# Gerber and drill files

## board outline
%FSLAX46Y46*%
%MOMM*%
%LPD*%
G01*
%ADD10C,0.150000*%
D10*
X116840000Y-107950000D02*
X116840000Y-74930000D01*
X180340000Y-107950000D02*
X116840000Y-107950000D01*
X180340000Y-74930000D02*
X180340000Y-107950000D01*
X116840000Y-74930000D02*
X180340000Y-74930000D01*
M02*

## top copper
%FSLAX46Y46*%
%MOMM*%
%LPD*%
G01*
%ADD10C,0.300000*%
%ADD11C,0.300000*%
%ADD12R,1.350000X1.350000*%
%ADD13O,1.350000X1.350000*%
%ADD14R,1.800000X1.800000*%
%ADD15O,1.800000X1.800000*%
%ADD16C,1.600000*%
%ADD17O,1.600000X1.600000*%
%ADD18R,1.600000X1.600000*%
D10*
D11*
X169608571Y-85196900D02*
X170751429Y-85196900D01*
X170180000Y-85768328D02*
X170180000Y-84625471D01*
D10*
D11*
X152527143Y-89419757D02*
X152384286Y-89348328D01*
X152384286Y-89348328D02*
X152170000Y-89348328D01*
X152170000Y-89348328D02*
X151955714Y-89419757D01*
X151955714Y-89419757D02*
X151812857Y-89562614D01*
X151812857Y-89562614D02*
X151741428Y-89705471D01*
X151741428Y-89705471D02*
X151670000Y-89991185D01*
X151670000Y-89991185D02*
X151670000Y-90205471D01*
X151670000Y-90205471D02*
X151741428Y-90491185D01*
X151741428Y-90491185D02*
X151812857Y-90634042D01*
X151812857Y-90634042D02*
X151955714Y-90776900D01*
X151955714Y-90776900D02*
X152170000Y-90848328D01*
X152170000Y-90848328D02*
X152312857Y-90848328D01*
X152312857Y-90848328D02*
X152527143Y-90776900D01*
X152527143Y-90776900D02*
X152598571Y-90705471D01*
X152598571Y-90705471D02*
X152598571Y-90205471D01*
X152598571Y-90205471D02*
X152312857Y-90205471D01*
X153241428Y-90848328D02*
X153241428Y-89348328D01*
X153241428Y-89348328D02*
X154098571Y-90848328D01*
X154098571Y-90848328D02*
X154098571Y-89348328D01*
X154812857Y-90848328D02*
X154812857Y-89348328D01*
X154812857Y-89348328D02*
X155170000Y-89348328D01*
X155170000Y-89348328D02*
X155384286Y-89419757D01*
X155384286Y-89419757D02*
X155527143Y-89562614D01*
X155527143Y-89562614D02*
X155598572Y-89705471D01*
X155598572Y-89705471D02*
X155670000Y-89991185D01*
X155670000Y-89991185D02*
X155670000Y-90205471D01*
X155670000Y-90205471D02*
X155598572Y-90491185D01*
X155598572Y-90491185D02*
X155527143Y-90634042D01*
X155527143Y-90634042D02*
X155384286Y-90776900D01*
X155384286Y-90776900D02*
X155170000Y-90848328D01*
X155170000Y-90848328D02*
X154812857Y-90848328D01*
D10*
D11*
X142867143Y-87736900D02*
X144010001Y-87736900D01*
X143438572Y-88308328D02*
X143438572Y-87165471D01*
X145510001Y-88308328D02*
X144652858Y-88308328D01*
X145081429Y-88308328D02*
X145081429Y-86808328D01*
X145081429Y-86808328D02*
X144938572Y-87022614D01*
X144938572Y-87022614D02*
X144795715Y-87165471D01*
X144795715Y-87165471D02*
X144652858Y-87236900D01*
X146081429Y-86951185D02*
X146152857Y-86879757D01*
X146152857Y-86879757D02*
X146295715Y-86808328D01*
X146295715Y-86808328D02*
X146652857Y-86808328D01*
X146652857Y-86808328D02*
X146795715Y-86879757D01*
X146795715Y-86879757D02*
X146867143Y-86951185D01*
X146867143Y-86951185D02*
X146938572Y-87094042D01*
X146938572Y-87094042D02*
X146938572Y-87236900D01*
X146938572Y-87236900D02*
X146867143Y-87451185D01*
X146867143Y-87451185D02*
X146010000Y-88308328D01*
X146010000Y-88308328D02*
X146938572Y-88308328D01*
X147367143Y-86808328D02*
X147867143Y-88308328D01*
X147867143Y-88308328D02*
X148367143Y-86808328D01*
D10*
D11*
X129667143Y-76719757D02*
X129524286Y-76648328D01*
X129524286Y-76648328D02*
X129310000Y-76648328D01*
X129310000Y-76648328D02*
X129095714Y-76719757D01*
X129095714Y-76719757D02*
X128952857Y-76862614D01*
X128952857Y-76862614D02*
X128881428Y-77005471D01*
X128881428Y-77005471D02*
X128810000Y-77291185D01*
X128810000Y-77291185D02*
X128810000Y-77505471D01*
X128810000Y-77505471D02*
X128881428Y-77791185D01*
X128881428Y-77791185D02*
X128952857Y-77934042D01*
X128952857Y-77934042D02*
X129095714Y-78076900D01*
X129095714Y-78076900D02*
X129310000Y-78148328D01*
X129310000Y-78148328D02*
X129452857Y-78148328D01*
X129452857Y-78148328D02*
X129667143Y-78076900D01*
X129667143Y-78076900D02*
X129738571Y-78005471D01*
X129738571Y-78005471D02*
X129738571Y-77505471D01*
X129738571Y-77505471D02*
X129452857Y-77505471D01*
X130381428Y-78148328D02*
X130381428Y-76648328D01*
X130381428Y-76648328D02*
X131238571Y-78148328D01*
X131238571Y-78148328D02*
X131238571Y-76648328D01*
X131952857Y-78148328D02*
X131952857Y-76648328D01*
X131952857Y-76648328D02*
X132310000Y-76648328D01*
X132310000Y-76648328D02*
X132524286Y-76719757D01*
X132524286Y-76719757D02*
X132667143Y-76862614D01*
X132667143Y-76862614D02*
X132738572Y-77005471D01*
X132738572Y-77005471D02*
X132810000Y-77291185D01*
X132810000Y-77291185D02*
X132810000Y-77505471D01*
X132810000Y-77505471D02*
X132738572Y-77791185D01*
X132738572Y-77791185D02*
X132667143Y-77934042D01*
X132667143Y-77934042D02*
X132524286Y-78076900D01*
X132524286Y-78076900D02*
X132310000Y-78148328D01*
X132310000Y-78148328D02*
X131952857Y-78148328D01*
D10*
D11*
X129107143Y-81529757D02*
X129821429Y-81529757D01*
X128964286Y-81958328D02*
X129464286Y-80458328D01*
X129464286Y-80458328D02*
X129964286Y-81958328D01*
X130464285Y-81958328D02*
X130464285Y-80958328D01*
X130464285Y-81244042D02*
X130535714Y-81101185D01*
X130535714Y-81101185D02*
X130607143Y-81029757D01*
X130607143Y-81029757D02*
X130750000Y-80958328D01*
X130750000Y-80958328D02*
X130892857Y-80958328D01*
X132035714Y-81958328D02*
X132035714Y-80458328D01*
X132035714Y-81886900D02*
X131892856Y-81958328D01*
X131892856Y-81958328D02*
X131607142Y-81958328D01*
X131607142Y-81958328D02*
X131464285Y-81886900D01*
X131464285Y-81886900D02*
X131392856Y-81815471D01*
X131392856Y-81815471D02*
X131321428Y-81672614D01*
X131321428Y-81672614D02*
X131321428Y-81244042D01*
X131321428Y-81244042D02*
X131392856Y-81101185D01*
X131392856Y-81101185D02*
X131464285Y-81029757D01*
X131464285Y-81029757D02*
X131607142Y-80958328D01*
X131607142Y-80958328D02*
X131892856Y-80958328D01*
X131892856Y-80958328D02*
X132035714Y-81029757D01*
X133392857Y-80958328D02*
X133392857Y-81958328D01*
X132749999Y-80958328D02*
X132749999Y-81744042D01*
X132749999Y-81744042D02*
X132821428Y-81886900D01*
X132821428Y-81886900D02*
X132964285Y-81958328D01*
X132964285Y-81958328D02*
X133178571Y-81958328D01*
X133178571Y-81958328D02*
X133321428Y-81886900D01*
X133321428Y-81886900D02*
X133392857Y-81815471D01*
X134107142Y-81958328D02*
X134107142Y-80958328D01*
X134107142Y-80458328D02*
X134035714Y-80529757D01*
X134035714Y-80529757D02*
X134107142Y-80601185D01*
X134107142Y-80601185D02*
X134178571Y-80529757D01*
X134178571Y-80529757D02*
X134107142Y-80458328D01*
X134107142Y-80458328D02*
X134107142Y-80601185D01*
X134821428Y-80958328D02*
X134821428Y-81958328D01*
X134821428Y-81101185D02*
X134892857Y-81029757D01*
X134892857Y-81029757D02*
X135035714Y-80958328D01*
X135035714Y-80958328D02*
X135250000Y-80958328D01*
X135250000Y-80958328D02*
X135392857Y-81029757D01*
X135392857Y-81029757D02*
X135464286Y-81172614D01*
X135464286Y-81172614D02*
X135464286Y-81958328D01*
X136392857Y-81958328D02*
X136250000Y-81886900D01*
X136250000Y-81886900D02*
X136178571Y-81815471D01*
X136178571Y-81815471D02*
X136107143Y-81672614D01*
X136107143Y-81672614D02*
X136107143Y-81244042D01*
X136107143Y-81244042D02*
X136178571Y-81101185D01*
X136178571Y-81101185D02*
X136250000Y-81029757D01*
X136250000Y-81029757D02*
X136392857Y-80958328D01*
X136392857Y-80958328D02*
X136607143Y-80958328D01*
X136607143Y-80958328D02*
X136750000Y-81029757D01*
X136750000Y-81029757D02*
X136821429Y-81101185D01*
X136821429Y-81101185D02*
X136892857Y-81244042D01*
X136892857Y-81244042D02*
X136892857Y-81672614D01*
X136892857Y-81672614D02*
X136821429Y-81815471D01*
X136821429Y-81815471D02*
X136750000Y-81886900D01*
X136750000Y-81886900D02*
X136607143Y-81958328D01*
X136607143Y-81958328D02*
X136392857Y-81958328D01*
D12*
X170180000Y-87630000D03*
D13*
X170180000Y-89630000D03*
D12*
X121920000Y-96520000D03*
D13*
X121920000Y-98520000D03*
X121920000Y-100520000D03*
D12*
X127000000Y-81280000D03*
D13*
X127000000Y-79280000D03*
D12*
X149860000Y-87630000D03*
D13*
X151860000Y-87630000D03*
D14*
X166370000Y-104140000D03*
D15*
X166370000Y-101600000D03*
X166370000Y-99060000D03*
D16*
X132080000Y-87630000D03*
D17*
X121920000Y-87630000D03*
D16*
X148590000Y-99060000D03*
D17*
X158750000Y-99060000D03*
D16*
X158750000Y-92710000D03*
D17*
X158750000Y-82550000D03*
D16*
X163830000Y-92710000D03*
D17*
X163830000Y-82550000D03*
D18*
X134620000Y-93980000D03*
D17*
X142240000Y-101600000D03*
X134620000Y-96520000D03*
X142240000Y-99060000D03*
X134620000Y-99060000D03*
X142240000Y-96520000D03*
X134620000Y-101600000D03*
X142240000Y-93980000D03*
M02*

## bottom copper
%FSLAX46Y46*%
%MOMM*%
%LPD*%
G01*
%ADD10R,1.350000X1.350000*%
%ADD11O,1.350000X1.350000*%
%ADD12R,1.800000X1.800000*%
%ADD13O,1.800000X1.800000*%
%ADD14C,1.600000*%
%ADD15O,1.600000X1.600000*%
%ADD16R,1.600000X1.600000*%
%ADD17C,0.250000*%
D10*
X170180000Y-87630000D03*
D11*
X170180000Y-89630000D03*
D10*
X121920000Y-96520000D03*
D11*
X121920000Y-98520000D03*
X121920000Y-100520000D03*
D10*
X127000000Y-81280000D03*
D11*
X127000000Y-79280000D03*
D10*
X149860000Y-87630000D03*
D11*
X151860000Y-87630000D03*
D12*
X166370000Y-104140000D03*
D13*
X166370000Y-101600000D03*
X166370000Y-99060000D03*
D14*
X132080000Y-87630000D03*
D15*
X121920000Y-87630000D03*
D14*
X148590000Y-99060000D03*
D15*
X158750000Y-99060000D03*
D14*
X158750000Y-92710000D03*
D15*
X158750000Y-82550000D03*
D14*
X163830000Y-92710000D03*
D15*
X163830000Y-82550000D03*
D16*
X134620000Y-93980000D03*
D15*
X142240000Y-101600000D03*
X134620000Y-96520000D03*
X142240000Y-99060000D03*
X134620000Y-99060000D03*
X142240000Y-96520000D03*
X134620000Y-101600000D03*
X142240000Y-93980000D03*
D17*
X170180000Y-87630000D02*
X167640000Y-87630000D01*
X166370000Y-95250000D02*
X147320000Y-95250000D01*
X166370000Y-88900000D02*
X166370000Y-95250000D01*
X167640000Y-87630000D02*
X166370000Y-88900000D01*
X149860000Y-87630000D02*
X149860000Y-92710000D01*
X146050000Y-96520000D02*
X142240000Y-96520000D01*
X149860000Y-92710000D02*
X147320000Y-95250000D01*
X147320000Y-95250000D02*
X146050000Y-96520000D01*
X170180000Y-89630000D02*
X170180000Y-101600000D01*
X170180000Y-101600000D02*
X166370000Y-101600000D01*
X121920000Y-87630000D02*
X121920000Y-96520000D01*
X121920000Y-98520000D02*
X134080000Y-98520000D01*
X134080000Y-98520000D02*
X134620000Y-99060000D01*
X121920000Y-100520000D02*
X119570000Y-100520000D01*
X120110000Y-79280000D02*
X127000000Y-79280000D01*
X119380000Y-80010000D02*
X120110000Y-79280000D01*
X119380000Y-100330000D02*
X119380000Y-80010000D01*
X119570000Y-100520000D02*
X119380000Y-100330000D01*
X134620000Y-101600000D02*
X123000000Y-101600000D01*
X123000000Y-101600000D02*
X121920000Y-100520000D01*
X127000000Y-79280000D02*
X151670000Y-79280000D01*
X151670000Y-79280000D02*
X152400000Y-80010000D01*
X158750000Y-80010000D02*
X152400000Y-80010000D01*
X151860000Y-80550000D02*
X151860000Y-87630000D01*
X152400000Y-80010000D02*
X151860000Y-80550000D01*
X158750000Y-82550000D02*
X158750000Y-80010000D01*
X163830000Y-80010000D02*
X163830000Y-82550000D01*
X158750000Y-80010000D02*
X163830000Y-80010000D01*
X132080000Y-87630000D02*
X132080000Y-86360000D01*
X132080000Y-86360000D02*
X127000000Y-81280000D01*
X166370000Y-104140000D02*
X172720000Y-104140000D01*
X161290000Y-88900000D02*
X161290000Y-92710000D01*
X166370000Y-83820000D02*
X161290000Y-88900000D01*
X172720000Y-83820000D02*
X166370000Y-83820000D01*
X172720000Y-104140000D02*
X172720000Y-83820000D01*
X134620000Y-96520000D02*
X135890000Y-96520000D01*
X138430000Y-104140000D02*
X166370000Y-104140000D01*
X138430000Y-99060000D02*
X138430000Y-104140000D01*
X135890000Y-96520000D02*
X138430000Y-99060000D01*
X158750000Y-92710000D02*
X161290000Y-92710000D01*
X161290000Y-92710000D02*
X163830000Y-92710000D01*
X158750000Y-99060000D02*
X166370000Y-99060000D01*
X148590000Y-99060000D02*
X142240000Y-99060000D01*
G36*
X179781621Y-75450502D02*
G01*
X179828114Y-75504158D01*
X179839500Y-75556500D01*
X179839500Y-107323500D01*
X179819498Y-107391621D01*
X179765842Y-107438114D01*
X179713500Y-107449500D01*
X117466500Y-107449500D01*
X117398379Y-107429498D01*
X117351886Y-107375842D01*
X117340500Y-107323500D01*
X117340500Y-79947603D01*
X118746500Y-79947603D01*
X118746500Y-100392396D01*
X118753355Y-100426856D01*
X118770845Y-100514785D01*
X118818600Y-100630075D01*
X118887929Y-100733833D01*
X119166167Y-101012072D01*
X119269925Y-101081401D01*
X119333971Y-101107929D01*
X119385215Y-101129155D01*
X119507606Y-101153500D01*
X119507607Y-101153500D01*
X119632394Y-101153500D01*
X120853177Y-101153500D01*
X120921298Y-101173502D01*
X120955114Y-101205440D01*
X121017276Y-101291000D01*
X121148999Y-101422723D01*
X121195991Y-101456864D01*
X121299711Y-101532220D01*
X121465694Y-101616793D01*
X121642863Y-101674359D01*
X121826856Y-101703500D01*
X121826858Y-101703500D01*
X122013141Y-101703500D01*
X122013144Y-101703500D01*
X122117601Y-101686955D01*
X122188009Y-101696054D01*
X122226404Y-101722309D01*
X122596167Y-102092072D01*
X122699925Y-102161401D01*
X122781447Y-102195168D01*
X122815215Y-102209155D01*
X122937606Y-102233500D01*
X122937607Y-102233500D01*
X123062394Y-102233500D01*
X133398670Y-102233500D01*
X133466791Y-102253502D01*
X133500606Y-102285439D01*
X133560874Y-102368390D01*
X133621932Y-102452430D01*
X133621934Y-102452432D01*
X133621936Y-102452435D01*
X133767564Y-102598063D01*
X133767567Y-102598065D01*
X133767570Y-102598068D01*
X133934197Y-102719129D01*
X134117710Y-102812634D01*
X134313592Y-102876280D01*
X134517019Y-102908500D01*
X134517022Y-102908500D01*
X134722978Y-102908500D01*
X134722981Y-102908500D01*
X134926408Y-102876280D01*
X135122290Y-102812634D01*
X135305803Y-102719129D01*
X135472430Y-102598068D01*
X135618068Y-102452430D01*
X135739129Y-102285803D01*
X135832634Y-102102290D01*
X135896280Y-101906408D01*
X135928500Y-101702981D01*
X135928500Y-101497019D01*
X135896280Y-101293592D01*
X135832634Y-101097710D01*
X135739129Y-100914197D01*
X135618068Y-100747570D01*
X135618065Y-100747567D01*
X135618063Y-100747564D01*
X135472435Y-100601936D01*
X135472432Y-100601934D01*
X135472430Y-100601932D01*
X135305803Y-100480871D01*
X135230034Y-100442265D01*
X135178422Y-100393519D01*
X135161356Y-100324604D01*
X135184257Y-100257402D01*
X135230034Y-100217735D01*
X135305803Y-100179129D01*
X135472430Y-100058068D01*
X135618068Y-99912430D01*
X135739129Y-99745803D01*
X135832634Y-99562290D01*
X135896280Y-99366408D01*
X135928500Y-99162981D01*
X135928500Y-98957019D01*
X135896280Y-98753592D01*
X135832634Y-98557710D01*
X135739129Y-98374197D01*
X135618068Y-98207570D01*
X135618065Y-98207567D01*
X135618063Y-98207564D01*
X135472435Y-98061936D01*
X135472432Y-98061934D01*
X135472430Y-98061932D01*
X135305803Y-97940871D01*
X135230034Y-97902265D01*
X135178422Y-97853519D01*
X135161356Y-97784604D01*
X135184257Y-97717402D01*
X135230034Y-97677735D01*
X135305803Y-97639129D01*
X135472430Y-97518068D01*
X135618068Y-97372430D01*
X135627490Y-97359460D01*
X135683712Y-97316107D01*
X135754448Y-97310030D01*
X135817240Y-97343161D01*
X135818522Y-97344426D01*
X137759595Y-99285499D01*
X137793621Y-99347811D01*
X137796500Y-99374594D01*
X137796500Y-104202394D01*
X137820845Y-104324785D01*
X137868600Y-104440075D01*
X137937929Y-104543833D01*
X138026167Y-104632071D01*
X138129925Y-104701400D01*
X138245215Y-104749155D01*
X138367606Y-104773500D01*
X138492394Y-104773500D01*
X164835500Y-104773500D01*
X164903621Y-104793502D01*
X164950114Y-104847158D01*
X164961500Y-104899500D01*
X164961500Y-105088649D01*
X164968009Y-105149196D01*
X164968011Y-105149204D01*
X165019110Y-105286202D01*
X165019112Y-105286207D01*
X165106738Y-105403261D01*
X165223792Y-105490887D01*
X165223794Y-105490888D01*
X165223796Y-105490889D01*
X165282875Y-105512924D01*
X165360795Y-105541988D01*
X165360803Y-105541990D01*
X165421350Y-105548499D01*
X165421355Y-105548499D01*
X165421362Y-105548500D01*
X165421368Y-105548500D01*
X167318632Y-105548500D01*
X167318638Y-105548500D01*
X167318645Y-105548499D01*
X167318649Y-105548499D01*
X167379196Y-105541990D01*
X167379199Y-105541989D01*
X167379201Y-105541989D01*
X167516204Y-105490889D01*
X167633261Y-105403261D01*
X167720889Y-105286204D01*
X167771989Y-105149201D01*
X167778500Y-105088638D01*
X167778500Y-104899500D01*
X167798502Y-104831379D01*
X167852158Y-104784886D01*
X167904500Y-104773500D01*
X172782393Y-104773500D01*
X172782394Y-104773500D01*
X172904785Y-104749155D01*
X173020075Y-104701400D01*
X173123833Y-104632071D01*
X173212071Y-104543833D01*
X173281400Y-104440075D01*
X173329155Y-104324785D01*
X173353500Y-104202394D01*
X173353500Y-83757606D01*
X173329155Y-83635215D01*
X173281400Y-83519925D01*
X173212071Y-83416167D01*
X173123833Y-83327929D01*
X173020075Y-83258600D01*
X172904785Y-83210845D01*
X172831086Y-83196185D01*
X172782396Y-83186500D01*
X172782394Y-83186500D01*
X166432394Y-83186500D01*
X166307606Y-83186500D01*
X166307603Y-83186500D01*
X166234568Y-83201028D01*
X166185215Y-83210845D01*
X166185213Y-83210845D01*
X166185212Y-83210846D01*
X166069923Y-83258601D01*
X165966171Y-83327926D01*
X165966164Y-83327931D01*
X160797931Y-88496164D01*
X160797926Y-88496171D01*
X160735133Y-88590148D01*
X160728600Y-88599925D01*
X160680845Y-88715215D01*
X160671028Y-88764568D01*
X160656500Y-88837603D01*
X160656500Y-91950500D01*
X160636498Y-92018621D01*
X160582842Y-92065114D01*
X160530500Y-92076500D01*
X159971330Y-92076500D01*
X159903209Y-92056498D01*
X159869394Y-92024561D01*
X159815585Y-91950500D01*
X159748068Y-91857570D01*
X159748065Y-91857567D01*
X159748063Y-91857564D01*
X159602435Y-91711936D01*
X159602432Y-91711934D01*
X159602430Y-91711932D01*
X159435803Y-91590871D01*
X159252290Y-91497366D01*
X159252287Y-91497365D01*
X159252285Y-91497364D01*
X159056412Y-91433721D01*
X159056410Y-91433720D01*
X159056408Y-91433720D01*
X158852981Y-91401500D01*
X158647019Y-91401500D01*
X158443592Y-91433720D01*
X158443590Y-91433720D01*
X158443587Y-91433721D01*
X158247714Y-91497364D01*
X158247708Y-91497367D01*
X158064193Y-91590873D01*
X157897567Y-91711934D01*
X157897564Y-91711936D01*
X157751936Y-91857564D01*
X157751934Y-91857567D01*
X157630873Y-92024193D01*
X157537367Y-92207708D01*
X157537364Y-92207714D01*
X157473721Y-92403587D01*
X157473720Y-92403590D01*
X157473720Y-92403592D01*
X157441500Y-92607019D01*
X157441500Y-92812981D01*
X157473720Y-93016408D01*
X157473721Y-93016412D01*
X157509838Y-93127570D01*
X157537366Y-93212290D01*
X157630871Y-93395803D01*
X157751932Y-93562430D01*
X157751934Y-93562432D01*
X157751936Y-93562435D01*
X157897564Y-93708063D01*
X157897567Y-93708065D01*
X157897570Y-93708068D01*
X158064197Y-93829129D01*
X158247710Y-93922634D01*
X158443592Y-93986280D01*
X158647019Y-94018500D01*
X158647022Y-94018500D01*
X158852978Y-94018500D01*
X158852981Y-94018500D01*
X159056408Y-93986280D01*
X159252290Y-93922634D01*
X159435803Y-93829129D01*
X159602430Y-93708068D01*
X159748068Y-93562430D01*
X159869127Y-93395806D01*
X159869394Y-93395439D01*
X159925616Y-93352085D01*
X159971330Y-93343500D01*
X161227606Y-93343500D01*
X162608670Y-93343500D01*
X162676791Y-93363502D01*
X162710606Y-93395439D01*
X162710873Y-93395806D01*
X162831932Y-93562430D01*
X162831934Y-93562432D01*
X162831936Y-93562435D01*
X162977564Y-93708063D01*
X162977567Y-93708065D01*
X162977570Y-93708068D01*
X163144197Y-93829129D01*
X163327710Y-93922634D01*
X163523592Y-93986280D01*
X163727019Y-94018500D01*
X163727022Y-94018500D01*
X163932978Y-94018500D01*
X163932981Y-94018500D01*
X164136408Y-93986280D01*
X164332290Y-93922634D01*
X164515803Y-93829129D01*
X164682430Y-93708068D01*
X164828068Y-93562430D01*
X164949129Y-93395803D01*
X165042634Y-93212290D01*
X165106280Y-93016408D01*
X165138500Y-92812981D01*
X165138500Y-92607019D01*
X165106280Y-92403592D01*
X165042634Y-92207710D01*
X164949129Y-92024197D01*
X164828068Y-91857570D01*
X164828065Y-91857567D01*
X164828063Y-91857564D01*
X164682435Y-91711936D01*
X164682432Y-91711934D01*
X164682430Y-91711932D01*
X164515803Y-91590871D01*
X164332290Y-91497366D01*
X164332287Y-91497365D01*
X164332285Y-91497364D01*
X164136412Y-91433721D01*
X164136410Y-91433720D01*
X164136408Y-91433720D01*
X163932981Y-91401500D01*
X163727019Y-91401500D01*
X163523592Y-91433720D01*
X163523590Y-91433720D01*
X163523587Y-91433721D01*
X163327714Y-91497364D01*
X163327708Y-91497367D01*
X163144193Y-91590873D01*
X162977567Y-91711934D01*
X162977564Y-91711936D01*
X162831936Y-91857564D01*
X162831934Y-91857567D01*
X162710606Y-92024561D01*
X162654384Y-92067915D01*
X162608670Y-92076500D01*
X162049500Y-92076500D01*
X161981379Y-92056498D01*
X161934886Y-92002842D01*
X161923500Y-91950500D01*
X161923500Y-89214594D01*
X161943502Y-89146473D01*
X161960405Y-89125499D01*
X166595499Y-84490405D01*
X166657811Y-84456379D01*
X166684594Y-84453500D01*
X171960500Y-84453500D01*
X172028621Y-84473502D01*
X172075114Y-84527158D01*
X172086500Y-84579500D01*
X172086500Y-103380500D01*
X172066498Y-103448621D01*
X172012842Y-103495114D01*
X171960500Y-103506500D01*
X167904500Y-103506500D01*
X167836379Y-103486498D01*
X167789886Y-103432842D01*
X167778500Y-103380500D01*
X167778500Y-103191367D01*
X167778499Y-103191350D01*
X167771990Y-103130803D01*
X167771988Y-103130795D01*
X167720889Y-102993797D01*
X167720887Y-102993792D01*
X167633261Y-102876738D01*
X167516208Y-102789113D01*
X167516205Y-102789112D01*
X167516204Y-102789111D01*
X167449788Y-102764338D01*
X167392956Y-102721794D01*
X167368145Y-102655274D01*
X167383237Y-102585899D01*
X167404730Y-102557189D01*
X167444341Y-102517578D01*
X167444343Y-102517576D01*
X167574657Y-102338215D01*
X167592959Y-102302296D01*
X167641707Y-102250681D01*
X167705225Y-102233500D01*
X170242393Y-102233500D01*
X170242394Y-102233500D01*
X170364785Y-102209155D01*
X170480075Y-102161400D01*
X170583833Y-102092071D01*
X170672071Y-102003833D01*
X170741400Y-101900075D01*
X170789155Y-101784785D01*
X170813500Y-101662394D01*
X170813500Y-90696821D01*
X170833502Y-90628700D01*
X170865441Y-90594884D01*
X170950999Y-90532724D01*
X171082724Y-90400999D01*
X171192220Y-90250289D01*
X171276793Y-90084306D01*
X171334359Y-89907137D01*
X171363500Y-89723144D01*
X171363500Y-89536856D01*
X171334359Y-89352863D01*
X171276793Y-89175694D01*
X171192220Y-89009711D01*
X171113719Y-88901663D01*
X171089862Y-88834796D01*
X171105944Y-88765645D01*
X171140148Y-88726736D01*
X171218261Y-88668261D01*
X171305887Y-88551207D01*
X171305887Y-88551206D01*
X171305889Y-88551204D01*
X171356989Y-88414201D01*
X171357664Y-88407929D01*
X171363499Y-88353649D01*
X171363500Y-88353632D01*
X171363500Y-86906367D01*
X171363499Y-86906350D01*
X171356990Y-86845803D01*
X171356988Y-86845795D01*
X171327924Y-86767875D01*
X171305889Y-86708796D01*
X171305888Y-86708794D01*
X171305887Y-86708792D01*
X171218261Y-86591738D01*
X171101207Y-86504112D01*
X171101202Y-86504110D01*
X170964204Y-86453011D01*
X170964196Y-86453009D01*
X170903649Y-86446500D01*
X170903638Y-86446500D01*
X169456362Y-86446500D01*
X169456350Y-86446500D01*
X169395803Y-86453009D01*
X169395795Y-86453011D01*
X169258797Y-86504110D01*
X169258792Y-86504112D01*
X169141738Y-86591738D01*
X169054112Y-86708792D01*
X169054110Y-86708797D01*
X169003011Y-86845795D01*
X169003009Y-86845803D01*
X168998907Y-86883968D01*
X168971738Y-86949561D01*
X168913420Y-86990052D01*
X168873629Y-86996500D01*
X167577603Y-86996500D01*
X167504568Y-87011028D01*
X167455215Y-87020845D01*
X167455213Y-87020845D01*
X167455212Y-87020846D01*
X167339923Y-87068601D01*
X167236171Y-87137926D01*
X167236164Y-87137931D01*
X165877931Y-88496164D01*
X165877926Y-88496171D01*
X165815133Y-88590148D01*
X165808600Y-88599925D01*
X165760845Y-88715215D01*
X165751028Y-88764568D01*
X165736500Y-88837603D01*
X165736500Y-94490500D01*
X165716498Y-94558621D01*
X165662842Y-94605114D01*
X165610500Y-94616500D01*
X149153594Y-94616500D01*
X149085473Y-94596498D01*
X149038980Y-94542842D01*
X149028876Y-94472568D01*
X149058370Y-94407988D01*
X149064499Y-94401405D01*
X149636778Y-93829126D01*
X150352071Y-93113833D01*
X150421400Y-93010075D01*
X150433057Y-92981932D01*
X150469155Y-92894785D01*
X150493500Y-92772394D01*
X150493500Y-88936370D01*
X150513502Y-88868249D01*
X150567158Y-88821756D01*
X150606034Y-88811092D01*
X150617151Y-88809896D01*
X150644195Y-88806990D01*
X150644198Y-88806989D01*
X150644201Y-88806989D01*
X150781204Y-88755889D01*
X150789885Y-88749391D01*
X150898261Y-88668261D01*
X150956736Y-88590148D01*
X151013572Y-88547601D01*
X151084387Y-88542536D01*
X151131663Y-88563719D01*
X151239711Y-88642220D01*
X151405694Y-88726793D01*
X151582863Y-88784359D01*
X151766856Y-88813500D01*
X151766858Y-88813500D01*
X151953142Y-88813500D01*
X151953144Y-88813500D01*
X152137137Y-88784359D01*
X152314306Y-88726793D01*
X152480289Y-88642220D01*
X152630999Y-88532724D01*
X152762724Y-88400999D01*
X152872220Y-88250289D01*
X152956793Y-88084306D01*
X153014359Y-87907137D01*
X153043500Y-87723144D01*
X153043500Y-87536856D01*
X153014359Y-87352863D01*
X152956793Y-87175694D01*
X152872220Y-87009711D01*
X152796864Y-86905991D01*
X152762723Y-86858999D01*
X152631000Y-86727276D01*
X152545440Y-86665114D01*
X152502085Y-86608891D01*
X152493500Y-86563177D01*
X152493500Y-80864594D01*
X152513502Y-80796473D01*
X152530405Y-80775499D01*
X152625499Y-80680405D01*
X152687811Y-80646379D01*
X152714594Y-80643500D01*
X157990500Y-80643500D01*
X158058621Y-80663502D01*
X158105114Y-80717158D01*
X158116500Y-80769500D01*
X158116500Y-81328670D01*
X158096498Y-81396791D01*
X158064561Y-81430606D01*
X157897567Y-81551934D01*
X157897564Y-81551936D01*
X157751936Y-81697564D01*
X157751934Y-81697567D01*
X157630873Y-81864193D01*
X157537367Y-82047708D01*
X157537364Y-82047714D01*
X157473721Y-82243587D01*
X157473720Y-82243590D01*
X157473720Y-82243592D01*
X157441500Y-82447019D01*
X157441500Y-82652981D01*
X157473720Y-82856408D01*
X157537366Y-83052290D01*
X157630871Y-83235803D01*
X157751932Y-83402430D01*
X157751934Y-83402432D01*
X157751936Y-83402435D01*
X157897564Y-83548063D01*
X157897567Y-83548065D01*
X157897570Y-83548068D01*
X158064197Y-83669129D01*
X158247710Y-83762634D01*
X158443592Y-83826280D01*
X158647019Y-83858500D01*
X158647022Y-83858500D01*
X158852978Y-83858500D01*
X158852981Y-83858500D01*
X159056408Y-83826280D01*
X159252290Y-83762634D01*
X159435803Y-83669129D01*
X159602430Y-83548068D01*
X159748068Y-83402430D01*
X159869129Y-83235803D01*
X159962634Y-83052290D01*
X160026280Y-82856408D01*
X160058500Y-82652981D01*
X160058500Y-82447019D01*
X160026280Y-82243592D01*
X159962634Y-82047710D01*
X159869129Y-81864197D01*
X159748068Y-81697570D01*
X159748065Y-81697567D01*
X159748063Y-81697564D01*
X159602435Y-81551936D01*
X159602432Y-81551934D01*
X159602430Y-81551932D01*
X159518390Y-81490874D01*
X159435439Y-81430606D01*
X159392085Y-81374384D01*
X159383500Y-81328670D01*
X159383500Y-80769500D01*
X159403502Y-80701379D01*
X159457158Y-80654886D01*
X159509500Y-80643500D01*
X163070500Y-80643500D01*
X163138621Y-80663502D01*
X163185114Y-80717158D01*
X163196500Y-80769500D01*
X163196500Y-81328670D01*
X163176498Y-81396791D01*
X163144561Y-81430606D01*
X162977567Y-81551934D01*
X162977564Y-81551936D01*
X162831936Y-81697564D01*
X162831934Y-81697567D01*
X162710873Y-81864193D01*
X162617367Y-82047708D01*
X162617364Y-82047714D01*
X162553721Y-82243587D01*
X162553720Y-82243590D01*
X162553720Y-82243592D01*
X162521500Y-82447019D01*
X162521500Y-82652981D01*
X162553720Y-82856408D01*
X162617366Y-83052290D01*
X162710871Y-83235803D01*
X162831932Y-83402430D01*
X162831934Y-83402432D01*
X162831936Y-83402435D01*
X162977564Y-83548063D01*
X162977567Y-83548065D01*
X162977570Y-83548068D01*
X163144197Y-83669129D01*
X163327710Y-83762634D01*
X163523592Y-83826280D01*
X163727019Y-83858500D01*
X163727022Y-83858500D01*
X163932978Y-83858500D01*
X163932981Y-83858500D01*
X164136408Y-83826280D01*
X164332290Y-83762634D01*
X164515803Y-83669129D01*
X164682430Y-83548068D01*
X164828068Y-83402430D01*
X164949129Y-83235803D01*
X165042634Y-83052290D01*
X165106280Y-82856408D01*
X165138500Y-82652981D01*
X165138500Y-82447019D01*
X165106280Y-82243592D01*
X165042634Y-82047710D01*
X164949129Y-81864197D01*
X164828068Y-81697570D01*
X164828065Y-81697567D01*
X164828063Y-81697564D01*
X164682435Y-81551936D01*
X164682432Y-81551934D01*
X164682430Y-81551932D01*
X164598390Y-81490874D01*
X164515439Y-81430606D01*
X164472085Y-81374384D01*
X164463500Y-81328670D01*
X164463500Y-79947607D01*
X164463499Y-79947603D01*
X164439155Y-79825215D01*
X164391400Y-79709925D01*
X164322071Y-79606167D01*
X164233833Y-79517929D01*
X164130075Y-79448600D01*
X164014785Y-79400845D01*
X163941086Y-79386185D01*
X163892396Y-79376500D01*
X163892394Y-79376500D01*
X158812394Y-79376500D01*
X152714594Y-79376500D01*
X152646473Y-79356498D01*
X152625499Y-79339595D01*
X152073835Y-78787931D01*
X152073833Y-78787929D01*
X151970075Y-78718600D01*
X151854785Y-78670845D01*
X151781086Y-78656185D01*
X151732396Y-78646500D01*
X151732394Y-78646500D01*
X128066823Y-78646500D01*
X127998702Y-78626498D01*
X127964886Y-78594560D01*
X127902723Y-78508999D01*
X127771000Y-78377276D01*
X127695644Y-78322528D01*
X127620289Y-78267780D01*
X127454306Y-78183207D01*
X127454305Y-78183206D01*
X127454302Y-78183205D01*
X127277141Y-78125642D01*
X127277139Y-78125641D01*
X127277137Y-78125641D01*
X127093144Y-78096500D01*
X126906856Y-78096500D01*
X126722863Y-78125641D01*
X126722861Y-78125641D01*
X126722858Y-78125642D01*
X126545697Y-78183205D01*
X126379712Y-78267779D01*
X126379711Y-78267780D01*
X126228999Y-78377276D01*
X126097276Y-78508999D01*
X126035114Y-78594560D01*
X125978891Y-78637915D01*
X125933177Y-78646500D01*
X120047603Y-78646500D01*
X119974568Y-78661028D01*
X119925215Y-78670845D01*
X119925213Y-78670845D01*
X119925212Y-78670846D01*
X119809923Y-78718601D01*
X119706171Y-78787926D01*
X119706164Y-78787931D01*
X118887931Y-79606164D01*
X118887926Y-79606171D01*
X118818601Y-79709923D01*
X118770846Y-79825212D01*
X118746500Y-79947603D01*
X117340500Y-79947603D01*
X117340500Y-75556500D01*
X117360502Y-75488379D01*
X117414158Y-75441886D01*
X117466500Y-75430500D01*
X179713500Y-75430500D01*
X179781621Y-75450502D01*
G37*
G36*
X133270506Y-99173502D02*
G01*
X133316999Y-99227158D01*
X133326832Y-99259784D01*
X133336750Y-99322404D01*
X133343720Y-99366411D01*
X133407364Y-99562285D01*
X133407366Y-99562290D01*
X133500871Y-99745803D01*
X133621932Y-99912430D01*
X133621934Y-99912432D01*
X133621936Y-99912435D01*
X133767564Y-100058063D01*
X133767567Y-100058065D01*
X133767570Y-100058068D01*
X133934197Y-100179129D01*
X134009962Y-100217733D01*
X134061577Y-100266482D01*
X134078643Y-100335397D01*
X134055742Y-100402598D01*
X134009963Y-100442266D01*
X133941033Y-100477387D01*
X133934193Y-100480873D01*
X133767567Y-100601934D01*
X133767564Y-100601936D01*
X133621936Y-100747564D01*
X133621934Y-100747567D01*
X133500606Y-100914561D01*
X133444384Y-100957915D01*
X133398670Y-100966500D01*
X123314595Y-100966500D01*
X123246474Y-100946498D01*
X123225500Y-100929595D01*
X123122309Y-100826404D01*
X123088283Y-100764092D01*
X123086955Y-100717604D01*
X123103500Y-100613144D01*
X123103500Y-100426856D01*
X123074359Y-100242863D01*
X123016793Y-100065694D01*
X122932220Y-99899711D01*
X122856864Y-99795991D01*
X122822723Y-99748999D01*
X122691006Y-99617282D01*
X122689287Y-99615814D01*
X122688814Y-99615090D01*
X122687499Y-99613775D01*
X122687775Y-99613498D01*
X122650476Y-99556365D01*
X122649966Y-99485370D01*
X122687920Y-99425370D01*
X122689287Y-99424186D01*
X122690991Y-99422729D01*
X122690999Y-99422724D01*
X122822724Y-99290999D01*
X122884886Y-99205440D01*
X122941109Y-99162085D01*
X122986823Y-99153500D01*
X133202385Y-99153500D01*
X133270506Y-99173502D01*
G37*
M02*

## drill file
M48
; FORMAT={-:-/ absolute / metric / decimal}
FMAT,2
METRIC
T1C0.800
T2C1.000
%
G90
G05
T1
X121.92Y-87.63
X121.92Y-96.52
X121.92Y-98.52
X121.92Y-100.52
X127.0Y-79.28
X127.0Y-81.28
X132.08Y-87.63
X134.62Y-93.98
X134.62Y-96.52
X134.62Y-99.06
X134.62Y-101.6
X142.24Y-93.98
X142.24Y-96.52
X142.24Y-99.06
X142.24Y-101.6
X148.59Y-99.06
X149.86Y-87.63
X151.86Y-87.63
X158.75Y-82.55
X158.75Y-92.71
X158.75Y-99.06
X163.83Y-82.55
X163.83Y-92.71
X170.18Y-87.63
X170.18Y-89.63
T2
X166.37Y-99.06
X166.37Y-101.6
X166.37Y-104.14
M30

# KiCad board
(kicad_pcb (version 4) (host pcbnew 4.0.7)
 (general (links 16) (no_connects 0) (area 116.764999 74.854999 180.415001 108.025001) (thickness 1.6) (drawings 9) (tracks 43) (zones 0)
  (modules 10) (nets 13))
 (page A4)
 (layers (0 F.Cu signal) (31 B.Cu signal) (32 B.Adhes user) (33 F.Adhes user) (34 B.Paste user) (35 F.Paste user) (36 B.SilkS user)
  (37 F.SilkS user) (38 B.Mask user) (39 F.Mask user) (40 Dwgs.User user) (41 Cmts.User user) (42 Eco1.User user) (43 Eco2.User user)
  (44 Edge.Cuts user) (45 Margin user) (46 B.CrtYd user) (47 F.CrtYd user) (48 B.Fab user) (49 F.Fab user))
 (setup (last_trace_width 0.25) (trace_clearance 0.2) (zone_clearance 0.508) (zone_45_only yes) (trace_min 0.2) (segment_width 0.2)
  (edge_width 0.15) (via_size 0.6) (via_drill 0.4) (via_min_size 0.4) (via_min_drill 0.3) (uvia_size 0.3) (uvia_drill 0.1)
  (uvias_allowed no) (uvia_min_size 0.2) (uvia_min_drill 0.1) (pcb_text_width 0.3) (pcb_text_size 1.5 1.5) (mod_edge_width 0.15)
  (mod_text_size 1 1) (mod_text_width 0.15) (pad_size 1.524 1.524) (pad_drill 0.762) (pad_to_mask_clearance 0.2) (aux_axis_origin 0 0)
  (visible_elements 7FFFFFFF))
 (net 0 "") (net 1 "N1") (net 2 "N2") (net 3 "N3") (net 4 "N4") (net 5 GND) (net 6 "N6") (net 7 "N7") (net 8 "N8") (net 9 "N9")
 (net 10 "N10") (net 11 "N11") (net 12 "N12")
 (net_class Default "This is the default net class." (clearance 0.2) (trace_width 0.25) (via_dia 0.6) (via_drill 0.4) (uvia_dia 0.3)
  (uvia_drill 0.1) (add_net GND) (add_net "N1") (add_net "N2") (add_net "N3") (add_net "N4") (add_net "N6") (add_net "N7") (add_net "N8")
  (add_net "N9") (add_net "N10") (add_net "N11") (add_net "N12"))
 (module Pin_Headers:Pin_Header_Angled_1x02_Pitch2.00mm (layer F.Cu) (at 170.18 87.63)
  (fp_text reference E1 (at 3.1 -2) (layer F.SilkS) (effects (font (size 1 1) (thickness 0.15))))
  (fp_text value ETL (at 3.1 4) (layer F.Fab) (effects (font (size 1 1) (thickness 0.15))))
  (pad 1 thru_hole rect (at 0 0) (size 1.35 1.35) (drill 0.8) (layers *.Cu *.Mask) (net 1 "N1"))
  (pad 2 thru_hole oval (at 0 2) (size 1.35 1.35) (drill 0.8) (layers *.Cu *.Mask) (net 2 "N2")))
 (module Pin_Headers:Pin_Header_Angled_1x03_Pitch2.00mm (layer F.Cu) (at 121.92 96.52)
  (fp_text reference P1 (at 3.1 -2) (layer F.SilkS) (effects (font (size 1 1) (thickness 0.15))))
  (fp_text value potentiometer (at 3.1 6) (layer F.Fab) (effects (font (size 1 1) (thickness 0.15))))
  (pad 1 thru_hole rect (at 0 0) (size 1.35 1.35) (drill 0.8) (layers *.Cu *.Mask) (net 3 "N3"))
  (pad 2 thru_hole oval (at 0 2) (size 1.35 1.35) (drill 0.8) (layers *.Cu *.Mask) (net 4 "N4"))
  (pad 3 thru_hole oval (at 0 4) (size 1.35 1.35) (drill 0.8) (layers *.Cu *.Mask) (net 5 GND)))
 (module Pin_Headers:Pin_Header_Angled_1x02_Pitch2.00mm (layer F.Cu) (at 127 81.28 180)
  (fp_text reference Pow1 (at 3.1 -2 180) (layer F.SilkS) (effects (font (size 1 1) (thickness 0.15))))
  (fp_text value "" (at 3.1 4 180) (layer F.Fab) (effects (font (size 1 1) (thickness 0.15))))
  (pad 1 thru_hole rect (at 0 0 180) (size 1.35 1.35) (drill 0.8) (layers *.Cu *.Mask) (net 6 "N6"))
  (pad 2 thru_hole oval (at 0 2 180) (size 1.35 1.35) (drill 0.8) (layers *.Cu *.Mask) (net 5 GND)))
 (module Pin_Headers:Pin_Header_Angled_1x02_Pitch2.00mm (layer F.Cu) (at 149.86 87.63 90)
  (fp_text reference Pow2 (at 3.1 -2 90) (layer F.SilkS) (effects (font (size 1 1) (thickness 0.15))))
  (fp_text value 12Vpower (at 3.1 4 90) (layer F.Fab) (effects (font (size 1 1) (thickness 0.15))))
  (pad 1 thru_hole rect (at 0 0 90) (size 1.35 1.35) (drill 0.8) (layers *.Cu *.Mask) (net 1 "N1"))
  (pad 2 thru_hole oval (at 0 2 90) (size 1.35 1.35) (drill 0.8) (layers *.Cu *.Mask) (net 5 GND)))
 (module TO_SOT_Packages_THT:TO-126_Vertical (layer F.Cu) (at 166.37 104.14 90)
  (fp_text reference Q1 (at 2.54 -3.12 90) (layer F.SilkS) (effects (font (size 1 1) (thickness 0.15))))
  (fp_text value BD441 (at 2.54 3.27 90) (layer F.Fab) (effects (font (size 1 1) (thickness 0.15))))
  (pad 1 thru_hole rect (at 0 0 90) (size 1.8 1.8) (drill 1) (layers *.Cu *.Mask) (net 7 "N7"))
  (pad 2 thru_hole oval (at 2.54 0 90) (size 1.8 1.8) (drill 1) (layers *.Cu *.Mask) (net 2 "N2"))
  (pad 3 thru_hole oval (at 5.08 0 90) (size 1.8 1.8) (drill 1) (layers *.Cu *.Mask) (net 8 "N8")))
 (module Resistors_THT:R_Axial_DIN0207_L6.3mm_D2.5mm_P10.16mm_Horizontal (layer F.Cu) (at 132.08 87.63 180)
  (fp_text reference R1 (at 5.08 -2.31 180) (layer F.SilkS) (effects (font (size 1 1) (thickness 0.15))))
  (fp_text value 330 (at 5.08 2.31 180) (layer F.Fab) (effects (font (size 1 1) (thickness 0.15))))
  (pad 1 thru_hole circle (at 0 0 180) (size 1.6 1.6) (drill 0.8) (layers *.Cu *.Mask) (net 6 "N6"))
  (pad 2 thru_hole oval (at 10.16 0 180) (size 1.6 1.6) (drill 0.8) (layers *.Cu *.Mask) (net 3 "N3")))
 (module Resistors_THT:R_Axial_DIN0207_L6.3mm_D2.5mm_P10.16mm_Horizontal (layer F.Cu) (at 148.59 99.06)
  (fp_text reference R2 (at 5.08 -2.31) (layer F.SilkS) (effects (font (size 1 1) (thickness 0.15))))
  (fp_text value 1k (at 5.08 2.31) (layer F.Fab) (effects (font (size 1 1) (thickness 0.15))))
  (pad 1 thru_hole circle (at 0 0) (size 1.6 1.6) (drill 0.8) (layers *.Cu *.Mask) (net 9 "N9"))
  (pad 2 thru_hole oval (at 10.16 0) (size 1.6 1.6) (drill 0.8) (layers *.Cu *.Mask) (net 8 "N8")))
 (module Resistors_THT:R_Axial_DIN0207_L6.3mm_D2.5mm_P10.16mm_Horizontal (layer F.Cu) (at 158.75 92.71 90)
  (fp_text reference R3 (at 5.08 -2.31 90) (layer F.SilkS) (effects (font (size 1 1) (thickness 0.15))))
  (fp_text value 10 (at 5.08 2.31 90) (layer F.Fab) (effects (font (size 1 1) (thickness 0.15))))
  (pad 1 thru_hole circle (at 0 0 90) (size 1.6 1.6) (drill 0.8) (layers *.Cu *.Mask) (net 7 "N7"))
  (pad 2 thru_hole oval (at 10.16 0 90) (size 1.6 1.6) (drill 0.8) (layers *.Cu *.Mask) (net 5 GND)))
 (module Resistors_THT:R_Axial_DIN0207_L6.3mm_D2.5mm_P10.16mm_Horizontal (layer F.Cu) (at 163.83 92.71 90)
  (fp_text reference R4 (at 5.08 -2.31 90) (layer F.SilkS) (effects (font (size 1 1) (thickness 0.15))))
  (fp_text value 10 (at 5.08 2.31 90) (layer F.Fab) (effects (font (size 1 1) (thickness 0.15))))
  (pad 1 thru_hole circle (at 0 0 90) (size 1.6 1.6) (drill 0.8) (layers *.Cu *.Mask) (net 7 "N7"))
  (pad 2 thru_hole oval (at 10.16 0 90) (size 1.6 1.6) (drill 0.8) (layers *.Cu *.Mask) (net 5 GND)))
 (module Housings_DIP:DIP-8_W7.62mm (layer F.Cu) (at 134.62 93.98)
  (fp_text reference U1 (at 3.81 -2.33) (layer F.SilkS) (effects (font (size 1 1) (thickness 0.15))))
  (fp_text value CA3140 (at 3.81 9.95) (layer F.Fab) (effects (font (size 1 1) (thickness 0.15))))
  (pad 1 thru_hole rect (at 0 0) (size 1.6 1.6) (drill 0.8) (layers *.Cu *.Mask) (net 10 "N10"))
  (pad 5 thru_hole oval (at 7.62 7.62) (size 1.6 1.6) (drill 0.8) (layers *.Cu *.Mask) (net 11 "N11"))
  (pad 2 thru_hole oval (at 0 2.54) (size 1.6 1.6) (drill 0.8) (layers *.Cu *.Mask) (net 7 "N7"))
  (pad 6 thru_hole oval (at 7.62 5.08) (size 1.6 1.6) (drill 0.8) (layers *.Cu *.Mask) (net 9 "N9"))
  (pad 3 thru_hole oval (at 0 5.08) (size 1.6 1.6) (drill 0.8) (layers *.Cu *.Mask) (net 4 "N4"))
  (pad 7 thru_hole oval (at 7.62 2.54) (size 1.6 1.6) (drill 0.8) (layers *.Cu *.Mask) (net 1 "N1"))
  (pad 4 thru_hole oval (at 0 7.62) (size 1.6 1.6) (drill 0.8) (layers *.Cu *.Mask) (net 5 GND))
  (pad 8 thru_hole oval (at 7.62 0) (size 1.6 1.6) (drill 0.8) (layers *.Cu *.Mask) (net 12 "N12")))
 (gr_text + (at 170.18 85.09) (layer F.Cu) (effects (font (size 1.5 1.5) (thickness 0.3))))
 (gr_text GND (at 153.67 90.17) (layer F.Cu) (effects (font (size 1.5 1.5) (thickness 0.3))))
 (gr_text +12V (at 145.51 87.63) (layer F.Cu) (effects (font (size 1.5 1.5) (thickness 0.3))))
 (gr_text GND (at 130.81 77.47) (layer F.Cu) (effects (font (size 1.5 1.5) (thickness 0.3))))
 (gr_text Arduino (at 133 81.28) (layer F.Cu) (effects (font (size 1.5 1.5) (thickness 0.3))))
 (gr_line (start 116.84 107.95) (end 116.84 74.93) (angle 90) (layer Edge.Cuts) (width 0.15))
 (gr_line (start 180.34 107.95) (end 116.84 107.95) (angle 90) (layer Edge.Cuts) (width 0.15))
 (gr_line (start 180.34 74.93) (end 180.34 107.95) (angle 90) (layer Edge.Cuts) (width 0.15))
 (gr_line (start 116.84 74.93) (end 180.34 74.93) (angle 90) (layer Edge.Cuts) (width 0.15))
 (segment (start 170.18 87.63) (end 167.64 87.63) (width 0.25) (layer B.Cu) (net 1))
 (segment (start 166.37 95.25) (end 147.32 95.25) (width 0.25) (layer B.Cu) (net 1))
 (segment (start 166.37 88.9) (end 166.37 95.25) (width 0.25) (layer B.Cu) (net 1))
 (segment (start 167.64 87.63) (end 166.37 88.9) (width 0.25) (layer B.Cu) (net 1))
 (segment (start 149.86 87.63) (end 149.86 92.71) (width 0.25) (layer B.Cu) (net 1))
 (segment (start 146.05 96.52) (end 142.24 96.52) (width 0.25) (layer B.Cu) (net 1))
 (segment (start 149.86 92.71) (end 147.32 95.25) (width 0.25) (layer B.Cu) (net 1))
 (segment (start 147.32 95.25) (end 146.05 96.52) (width 0.25) (layer B.Cu) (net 1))
 (segment (start 170.18 89.63) (end 170.18 101.6) (width 0.25) (layer B.Cu) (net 2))
 (segment (start 170.18 101.6) (end 166.37 101.6) (width 0.25) (layer B.Cu) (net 2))
 (segment (start 121.92 87.63) (end 121.92 96.52) (width 0.25) (layer B.Cu) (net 3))
 (segment (start 121.92 98.52) (end 134.08 98.52) (width 0.25) (layer B.Cu) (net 4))
 (segment (start 134.08 98.52) (end 134.62 99.06) (width 0.25) (layer B.Cu) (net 4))
 (segment (start 121.92 100.52) (end 119.57 100.52) (width 0.25) (layer B.Cu) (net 5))
 (segment (start 120.11 79.28) (end 127 79.28) (width 0.25) (layer B.Cu) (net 5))
 (segment (start 119.38 80.01) (end 120.11 79.28) (width 0.25) (layer B.Cu) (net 5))
 (segment (start 119.38 100.33) (end 119.38 80.01) (width 0.25) (layer B.Cu) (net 5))
 (segment (start 119.57 100.52) (end 119.38 100.33) (width 0.25) (layer B.Cu) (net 5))
 (segment (start 134.62 101.6) (end 123 101.6) (width 0.25) (layer B.Cu) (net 5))
 (segment (start 123 101.6) (end 121.92 100.52) (width 0.25) (layer B.Cu) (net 5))
 (segment (start 127 79.28) (end 151.67 79.28) (width 0.25) (layer B.Cu) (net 5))
 (segment (start 151.67 79.28) (end 152.4 80.01) (width 0.25) (layer B.Cu) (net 5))
 (segment (start 158.75 80.01) (end 152.4 80.01) (width 0.25) (layer B.Cu) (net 5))
 (segment (start 151.86 80.55) (end 151.86 87.63) (width 0.25) (layer B.Cu) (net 5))
 (segment (start 152.4 80.01) (end 151.86 80.55) (width 0.25) (layer B.Cu) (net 5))
 (segment (start 158.75 82.55) (end 158.75 80.01) (width 0.25) (layer B.Cu) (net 5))
 (segment (start 163.83 80.01) (end 163.83 82.55) (width 0.25) (layer B.Cu) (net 5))
 (segment (start 158.75 80.01) (end 163.83 80.01) (width 0.25) (layer B.Cu) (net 5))
 (segment (start 132.08 87.63) (end 132.08 86.36) (width 0.25) (layer B.Cu) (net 6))
 (segment (start 132.08 86.36) (end 127 81.28) (width 0.25) (layer B.Cu) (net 6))
 (segment (start 166.37 104.14) (end 172.72 104.14) (width 0.25) (layer B.Cu) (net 7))
 (segment (start 161.29 88.9) (end 161.29 92.71) (width 0.25) (layer B.Cu) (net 7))
 (segment (start 166.37 83.82) (end 161.29 88.9) (width 0.25) (layer B.Cu) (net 7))
 (segment (start 172.72 83.82) (end 166.37 83.82) (width 0.25) (layer B.Cu) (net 7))
 (segment (start 172.72 104.14) (end 172.72 83.82) (width 0.25) (layer B.Cu) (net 7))
 (segment (start 134.62 96.52) (end 135.89 96.52) (width 0.25) (layer B.Cu) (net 7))
 (segment (start 138.43 104.14) (end 166.37 104.14) (width 0.25) (layer B.Cu) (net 7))
 (segment (start 138.43 99.06) (end 138.43 104.14) (width 0.25) (layer B.Cu) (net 7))
 (segment (start 135.89 96.52) (end 138.43 99.06) (width 0.25) (layer B.Cu) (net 7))
 (segment (start 158.75 92.71) (end 161.29 92.71) (width 0.25) (layer B.Cu) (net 7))
 (segment (start 161.29 92.71) (end 163.83 92.71) (width 0.25) (layer B.Cu) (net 7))
 (segment (start 158.75 99.06) (end 166.37 99.06) (width 0.25) (layer B.Cu) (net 8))
 (segment (start 148.59 99.06) (end 142.24 99.06) (width 0.25) (layer B.Cu) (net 9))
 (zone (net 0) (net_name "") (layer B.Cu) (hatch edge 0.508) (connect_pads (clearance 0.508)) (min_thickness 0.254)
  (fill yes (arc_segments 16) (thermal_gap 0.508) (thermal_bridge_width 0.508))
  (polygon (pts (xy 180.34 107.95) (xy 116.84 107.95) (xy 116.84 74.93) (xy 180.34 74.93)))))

